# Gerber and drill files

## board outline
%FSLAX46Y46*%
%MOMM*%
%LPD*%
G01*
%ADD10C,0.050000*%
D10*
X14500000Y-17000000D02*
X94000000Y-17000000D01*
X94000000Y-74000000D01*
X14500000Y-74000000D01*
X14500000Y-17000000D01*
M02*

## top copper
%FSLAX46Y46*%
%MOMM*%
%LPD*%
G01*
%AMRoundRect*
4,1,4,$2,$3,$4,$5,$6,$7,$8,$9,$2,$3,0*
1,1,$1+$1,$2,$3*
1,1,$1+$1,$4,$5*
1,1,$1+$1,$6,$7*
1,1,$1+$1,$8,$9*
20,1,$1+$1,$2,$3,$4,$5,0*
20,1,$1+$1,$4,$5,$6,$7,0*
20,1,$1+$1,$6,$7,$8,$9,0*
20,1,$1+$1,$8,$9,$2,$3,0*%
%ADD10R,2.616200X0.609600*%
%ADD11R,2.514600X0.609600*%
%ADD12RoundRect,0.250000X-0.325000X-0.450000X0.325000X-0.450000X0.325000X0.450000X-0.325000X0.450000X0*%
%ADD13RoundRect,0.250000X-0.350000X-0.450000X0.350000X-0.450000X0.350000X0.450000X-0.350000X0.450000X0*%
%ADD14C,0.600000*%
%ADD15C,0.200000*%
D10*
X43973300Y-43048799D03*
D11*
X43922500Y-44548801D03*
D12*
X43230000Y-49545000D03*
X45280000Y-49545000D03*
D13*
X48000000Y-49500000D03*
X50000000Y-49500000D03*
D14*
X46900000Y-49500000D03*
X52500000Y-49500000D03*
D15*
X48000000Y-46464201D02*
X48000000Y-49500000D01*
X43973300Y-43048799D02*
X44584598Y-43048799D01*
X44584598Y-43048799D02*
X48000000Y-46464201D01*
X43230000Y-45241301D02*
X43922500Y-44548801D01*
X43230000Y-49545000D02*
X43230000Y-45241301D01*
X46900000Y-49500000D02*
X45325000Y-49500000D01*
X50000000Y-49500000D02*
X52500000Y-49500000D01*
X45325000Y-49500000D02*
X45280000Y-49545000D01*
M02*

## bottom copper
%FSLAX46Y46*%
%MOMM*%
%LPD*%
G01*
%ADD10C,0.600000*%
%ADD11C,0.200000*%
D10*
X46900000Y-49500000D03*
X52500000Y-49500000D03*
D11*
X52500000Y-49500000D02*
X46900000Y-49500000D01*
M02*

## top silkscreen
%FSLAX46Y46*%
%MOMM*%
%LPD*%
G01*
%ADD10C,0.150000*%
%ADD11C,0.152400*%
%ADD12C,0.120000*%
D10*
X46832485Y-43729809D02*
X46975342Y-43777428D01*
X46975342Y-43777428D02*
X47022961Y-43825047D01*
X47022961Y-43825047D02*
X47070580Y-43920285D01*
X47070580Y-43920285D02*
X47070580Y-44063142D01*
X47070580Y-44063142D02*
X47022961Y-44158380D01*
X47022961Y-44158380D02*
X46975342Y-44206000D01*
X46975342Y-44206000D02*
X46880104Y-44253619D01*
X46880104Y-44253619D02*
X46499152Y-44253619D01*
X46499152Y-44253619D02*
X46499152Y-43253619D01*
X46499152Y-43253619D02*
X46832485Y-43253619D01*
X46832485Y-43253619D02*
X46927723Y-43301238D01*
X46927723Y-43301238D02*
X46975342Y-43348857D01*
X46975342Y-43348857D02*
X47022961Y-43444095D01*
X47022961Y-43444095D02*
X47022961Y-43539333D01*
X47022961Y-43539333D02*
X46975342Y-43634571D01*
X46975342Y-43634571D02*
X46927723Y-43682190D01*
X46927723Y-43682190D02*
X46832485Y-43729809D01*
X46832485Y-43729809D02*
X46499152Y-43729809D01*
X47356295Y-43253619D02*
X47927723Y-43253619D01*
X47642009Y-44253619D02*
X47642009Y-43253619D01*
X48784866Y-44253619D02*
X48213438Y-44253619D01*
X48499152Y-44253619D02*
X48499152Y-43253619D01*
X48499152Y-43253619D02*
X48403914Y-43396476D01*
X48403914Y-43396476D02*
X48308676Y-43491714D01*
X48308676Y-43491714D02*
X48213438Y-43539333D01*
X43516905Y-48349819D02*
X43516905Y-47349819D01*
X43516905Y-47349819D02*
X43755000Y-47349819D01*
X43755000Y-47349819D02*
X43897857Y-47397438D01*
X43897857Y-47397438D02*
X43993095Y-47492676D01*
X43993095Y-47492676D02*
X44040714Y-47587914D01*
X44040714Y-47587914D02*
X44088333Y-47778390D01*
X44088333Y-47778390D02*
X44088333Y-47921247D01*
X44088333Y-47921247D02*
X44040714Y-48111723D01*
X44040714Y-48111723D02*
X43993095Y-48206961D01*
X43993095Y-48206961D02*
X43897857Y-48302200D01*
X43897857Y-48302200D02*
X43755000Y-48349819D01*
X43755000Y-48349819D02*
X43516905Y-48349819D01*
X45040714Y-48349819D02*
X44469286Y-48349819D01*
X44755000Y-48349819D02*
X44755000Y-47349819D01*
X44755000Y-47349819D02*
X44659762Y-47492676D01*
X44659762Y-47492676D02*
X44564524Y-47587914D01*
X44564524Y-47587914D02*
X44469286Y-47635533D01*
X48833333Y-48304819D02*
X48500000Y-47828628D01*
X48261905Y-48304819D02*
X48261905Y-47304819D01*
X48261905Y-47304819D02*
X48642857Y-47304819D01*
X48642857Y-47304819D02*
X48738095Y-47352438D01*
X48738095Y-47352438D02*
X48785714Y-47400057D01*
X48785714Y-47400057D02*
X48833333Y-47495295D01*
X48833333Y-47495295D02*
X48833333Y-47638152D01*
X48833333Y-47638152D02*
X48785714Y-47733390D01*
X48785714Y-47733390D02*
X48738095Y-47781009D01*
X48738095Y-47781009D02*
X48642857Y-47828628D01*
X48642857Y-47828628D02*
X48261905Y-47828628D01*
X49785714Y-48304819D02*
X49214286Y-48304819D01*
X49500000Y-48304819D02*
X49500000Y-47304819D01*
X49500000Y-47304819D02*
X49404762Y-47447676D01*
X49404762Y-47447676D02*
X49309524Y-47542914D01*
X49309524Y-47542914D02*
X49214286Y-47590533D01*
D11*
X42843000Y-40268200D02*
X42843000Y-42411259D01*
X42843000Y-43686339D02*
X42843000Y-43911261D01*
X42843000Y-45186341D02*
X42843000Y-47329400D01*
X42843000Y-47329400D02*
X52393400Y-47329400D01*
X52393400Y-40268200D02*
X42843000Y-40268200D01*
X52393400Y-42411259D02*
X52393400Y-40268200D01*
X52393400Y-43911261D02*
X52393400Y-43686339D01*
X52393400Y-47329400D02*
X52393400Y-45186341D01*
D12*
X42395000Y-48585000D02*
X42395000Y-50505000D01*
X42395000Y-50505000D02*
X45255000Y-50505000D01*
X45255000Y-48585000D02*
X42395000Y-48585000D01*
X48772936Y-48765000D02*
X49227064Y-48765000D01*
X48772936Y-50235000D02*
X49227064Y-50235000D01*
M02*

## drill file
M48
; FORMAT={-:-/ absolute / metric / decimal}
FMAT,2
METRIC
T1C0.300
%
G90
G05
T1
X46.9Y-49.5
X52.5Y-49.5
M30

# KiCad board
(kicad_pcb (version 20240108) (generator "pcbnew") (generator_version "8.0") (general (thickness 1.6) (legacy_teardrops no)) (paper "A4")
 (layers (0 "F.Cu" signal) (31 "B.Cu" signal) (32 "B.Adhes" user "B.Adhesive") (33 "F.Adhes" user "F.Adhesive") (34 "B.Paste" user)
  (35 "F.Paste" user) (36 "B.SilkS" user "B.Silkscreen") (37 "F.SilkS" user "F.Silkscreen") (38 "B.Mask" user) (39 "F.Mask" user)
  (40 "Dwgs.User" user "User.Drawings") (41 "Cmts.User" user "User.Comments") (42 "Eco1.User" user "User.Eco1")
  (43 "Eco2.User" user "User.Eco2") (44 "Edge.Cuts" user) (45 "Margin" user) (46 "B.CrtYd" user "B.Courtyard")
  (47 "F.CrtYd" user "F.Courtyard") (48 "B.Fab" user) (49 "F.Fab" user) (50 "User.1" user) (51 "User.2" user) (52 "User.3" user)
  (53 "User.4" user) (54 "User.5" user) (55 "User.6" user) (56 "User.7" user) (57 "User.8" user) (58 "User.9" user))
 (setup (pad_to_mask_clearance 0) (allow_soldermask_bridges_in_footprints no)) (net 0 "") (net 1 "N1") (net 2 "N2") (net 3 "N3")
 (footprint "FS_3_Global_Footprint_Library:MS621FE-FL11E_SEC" (layer "F.Cu") (at 47.6182 43.7988)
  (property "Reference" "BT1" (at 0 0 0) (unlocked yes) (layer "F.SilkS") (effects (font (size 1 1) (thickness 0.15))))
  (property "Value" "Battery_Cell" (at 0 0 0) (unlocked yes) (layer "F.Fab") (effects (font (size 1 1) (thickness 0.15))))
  (fp_line (start -4.7752 -3.5306) (end -4.7752 -1.387541) (stroke (width 0.1524) (type solid)) (layer "F.SilkS"))
  (fp_line (start -4.7752 -0.112461) (end -4.7752 0.112461) (stroke (width 0.1524) (type solid)) (layer "F.SilkS"))
  (fp_line (start -4.7752 1.387541) (end -4.7752 3.5306) (stroke (width 0.1524) (type solid)) (layer "F.SilkS"))
  (fp_line (start -4.7752 3.5306) (end 4.7752 3.5306) (stroke (width 0.1524) (type solid)) (layer "F.SilkS"))
  (fp_line (start 4.7752 -3.5306) (end -4.7752 -3.5306) (stroke (width 0.1524) (type solid)) (layer "F.SilkS"))
  (fp_line (start 4.7752 -1.387541) (end 4.7752 -3.5306) (stroke (width 0.1524) (type solid)) (layer "F.SilkS"))
  (fp_line (start 4.7752 0.112461) (end 4.7752 -0.112461) (stroke (width 0.1524) (type solid)) (layer "F.SilkS"))
  (fp_line (start 4.7752 3.5306) (end 4.7752 1.387541) (stroke (width 0.1524) (type solid)) (layer "F.SilkS"))
  (pad "1" smd rect (at -3.6449 -0.750001) (size 2.6162 0.6096) (layers "F.Cu" "F.Paste" "F.Mask") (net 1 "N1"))
  (pad "2" smd rect (at -3.6957 0.750001) (size 2.5146 0.6096) (layers "F.Cu" "F.Paste" "F.Mask") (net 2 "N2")))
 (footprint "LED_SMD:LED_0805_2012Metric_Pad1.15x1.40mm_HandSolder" (layer "F.Cu") (at 44.255 49.545)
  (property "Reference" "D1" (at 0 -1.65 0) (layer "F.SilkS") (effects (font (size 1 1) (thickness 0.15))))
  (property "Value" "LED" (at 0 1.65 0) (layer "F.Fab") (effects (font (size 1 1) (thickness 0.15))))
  (fp_line (start -1.86 -0.96) (end -1.86 0.96) (stroke (width 0.12) (type solid)) (layer "F.SilkS"))
  (fp_line (start -1.86 0.96) (end 1 0.96) (stroke (width 0.12) (type solid)) (layer "F.SilkS"))
  (fp_line (start 1 -0.96) (end -1.86 -0.96) (stroke (width 0.12) (type solid)) (layer "F.SilkS"))
  (pad "1" smd roundrect (at -1.025 0) (size 1.15 1.4) (layers "F.Cu" "F.Paste" "F.Mask") (roundrect_rratio 0.217391) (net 2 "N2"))
  (pad "2" smd roundrect (at 1.025 0) (size 1.15 1.4) (layers "F.Cu" "F.Paste" "F.Mask") (roundrect_rratio 0.217391) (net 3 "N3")))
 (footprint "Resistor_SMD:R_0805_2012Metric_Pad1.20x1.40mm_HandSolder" (layer "F.Cu") (at 49 49.5)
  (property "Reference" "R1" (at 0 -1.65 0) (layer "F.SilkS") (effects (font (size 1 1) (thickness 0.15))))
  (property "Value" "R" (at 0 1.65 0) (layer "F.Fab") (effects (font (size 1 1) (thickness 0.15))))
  (fp_line (start -0.227064 -0.735) (end 0.227064 -0.735) (stroke (width 0.12) (type solid)) (layer "F.SilkS"))
  (fp_line (start -0.227064 0.735) (end 0.227064 0.735) (stroke (width 0.12) (type solid)) (layer "F.SilkS"))
  (pad "1" smd roundrect (at -1 0) (size 1.2 1.4) (layers "F.Cu" "F.Paste" "F.Mask") (roundrect_rratio 0.208333) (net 1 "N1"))
  (pad "2" smd roundrect (at 1 0) (size 1.2 1.4) (layers "F.Cu" "F.Paste" "F.Mask") (roundrect_rratio 0.208333) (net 3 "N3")))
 (gr_rect (start 14.5 17) (end 94 74) (stroke (width 0.05) (type default)) (fill none) (layer "Edge.Cuts"))
 (segment (start 48 46.464201) (end 48 49.5) (width 0.2) (layer "F.Cu") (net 1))
 (segment (start 43.9733 43.048799) (end 44.584598 43.048799) (width 0.2) (layer "F.Cu") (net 1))
 (segment (start 44.584598 43.048799) (end 48 46.464201) (width 0.2) (layer "F.Cu") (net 1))
 (segment (start 43.23 45.241301) (end 43.9225 44.548801) (width 0.2) (layer "F.Cu") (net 2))
 (segment (start 43.23 49.545) (end 43.23 45.241301) (width 0.2) (layer "F.Cu") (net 2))
 (segment (start 46.9 49.5) (end 45.325 49.5) (width 0.2) (layer "F.Cu") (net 3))
 (segment (start 50 49.5) (end 52.5 49.5) (width 0.2) (layer "F.Cu") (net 3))
 (segment (start 45.325 49.5) (end 45.28 49.545) (width 0.2) (layer "F.Cu") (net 3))
 (via (at 46.9 49.5) (size 0.6) (drill 0.3) (layers "F.Cu" "B.Cu") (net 3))
 (via (at 52.5 49.5) (size 0.6) (drill 0.3) (layers "F.Cu" "B.Cu") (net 3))
 (segment (start 52.5 49.5) (end 46.9 49.5) (width 0.2) (layer "B.Cu") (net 3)))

